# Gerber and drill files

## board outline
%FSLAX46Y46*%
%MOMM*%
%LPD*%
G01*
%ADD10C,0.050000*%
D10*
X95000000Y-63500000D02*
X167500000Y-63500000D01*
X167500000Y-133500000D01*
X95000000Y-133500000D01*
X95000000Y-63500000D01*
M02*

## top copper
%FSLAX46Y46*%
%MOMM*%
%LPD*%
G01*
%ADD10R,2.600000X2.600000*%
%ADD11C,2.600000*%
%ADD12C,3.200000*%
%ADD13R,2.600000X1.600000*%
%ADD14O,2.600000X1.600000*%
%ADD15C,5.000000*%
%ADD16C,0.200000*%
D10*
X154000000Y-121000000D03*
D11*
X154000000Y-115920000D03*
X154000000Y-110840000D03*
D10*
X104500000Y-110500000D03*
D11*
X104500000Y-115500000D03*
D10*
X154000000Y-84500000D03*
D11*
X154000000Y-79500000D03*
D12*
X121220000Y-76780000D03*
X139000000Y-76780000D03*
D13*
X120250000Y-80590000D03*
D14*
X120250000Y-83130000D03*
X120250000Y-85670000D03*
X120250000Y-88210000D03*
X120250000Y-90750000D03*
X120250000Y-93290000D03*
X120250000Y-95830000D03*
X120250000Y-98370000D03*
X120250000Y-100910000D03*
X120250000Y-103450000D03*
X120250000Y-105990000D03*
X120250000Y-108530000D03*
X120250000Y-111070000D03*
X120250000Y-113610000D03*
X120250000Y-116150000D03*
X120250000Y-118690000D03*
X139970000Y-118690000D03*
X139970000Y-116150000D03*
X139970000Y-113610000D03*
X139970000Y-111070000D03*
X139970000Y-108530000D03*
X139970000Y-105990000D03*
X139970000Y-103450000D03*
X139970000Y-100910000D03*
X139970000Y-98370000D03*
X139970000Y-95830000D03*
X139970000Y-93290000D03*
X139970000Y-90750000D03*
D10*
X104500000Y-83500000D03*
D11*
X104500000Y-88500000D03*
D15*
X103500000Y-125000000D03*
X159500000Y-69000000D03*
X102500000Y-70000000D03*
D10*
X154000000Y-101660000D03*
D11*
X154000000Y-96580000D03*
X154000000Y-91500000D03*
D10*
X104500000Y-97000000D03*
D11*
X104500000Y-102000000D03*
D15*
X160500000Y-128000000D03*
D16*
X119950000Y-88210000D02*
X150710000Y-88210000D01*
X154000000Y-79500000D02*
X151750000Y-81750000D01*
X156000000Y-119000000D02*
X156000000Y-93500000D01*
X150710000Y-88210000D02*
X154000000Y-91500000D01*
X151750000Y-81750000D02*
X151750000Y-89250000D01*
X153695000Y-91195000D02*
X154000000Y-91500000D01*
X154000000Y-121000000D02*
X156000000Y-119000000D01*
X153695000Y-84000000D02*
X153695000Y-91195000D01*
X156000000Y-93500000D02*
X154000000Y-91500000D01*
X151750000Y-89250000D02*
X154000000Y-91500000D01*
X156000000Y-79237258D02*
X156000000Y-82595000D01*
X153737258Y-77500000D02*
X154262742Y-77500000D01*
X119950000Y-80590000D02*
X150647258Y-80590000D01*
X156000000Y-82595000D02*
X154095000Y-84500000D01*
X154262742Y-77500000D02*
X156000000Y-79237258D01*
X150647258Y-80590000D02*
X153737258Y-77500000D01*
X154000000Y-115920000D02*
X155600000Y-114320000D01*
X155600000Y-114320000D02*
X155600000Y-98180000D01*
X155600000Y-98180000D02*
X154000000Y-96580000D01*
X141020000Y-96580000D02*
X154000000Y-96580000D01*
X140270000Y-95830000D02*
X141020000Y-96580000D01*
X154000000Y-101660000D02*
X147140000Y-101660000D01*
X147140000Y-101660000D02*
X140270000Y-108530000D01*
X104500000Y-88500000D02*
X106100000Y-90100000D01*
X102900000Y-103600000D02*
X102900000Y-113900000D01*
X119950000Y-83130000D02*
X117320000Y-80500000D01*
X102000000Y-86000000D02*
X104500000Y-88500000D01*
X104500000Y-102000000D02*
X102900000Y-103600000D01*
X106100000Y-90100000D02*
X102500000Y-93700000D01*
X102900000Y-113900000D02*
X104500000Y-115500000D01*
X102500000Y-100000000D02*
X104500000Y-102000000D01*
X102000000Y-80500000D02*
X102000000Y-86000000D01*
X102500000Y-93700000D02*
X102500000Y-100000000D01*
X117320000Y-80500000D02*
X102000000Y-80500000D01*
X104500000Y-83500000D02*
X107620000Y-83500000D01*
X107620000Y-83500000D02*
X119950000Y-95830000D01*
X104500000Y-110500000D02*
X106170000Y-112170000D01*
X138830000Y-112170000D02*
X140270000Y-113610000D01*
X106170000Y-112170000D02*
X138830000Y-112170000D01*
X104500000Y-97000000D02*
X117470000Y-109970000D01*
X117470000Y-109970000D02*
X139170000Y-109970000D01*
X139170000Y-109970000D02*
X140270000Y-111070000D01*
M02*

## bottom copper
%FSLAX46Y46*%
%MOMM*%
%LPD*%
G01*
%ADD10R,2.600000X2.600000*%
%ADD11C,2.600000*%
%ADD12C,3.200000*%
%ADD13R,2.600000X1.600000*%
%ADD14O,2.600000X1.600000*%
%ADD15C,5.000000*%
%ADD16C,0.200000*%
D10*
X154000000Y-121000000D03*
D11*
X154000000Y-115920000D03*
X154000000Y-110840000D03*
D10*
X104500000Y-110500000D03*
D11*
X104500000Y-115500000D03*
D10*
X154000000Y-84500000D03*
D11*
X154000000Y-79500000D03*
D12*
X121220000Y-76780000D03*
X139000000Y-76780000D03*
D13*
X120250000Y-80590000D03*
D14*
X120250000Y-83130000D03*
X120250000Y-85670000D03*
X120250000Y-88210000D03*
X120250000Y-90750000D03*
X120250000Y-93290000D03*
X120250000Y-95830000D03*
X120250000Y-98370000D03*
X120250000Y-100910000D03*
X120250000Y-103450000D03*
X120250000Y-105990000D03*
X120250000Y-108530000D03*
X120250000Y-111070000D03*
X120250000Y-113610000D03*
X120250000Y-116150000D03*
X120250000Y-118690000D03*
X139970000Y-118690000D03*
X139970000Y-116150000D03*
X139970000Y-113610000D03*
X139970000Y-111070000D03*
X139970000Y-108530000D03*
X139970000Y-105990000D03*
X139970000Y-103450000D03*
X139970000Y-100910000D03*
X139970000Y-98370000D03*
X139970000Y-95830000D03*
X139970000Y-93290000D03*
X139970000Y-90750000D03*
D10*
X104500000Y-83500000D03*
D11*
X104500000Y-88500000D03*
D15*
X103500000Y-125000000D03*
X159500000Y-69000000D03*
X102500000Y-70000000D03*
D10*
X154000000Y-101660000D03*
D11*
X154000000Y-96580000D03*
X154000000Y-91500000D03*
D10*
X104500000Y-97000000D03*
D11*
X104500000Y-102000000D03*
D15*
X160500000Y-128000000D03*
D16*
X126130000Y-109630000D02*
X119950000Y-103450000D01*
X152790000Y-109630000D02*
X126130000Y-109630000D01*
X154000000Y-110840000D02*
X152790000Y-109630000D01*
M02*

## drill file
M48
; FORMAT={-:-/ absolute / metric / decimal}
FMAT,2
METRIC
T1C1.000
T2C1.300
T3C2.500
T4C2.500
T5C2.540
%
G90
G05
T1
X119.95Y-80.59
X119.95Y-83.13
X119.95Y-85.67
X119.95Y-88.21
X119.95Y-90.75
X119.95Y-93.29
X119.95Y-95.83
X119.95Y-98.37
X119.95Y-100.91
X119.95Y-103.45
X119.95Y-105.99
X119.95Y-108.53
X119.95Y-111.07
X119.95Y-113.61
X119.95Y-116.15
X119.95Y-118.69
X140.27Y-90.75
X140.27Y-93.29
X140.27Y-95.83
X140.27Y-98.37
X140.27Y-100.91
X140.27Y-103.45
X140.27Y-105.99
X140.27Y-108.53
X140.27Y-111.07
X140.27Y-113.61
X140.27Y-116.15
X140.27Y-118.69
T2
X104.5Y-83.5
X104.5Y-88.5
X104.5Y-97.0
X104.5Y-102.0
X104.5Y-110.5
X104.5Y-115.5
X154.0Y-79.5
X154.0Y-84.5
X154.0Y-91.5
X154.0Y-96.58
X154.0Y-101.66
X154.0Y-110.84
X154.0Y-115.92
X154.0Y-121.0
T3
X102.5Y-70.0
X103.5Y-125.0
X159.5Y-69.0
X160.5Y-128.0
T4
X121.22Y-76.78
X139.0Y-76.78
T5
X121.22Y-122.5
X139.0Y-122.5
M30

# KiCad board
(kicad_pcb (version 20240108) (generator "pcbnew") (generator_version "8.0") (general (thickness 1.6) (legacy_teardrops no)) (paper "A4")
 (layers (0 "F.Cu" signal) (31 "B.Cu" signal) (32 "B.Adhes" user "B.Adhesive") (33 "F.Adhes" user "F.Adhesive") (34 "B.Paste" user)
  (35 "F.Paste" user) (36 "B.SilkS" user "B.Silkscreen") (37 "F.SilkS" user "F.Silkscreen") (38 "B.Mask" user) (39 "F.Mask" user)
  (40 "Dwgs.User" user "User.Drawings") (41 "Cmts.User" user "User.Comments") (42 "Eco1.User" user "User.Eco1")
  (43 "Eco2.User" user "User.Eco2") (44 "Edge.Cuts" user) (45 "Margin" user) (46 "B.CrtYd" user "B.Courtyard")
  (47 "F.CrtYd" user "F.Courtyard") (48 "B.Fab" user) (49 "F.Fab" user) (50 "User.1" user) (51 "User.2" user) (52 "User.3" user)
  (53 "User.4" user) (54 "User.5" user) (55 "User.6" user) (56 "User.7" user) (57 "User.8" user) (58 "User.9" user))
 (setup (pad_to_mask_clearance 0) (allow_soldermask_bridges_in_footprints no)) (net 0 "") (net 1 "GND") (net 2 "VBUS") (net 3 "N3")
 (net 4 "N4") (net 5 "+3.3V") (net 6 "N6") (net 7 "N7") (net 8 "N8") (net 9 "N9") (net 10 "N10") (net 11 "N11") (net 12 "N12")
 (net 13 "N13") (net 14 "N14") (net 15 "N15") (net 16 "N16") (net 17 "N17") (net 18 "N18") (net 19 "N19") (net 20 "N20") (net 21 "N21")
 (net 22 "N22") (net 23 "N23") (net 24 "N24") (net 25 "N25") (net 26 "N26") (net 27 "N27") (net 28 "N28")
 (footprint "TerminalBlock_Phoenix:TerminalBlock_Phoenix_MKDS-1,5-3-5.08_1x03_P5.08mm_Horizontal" (layer "F.Cu") (at 154 121 90)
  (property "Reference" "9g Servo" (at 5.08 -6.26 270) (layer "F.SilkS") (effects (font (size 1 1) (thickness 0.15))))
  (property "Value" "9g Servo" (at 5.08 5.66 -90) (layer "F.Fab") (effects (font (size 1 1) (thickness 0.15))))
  (pad "1" thru_hole rect (at 0 0 90) (size 2.6 2.6) (drill 1.3) (layers "*.Cu" "*.Mask") (remove_unused_layers no) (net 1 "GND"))
  (pad "2" thru_hole circle (at 5.08 0 90) (size 2.6 2.6) (drill 1.3) (layers "*.Cu" "*.Mask") (remove_unused_layers no) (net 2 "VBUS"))
  (pad "3" thru_hole circle (at 10.16 0 90) (size 2.6 2.6) (drill 1.3) (layers "*.Cu" "*.Mask") (remove_unused_layers no) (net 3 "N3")))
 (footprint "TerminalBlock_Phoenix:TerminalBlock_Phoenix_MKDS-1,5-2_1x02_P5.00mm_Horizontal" (layer "F.Cu") (at 104.5 110.5 -90)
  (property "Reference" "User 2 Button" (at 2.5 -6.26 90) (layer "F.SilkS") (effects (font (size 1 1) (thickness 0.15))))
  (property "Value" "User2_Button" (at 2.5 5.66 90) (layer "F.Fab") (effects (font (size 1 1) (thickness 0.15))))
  (pad "1" thru_hole rect (at 0 0 270) (size 2.6 2.6) (drill 1.3) (layers "*.Cu" "*.Mask") (remove_unused_layers no) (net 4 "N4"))
  (pad "2" thru_hole circle (at 5 0 270) (size 2.6 2.6) (drill 1.3) (layers "*.Cu" "*.Mask") (remove_unused_layers no) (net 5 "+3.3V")))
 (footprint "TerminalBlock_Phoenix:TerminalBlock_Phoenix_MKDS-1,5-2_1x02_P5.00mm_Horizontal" (layer "F.Cu") (at 154 84.5 90)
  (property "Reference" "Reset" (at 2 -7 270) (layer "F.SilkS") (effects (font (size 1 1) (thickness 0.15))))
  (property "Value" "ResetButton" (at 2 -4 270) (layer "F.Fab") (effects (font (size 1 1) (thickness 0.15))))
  (pad "1" thru_hole rect (at 0 0 90) (size 2.6 2.6) (drill 1.3) (layers "*.Cu" "*.Mask") (remove_unused_layers no) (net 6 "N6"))
  (pad "2" thru_hole circle (at 5 0 90) (size 2.6 2.6) (drill 1.3) (layers "*.Cu" "*.Mask") (remove_unused_layers no) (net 1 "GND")))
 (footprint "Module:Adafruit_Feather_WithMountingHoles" (layer "F.Cu") (at 119.95 80.59)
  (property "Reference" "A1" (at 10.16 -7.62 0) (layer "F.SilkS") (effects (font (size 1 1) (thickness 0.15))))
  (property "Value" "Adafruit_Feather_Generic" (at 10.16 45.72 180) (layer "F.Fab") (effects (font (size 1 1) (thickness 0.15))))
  (pad "" np_thru_hole circle (at 1.27 -3.81 270) (size 3.2 3.2) (drill 2.5) (layers "*.Cu" "*.Mask"))
  (pad "" np_thru_hole circle (at 1.27 41.91 270) (size 2.54 2.54) (drill 2.54) (layers "*.Cu" "*.Mask"))
  (pad "" np_thru_hole circle (at 19.05 -3.81 270) (size 3.2 3.2) (drill 2.5) (layers "*.Cu" "*.Mask"))
  (pad "" np_thru_hole circle (at 19.05 41.91 270) (size 2.54 2.54) (drill 2.54) (layers "*.Cu" "*.Mask"))
  (pad "1" thru_hole rect (at 0 0) (size 2.6 1.6) (drill 1 (offset 0.3 0)) (layers "*.Cu" "*.Mask") (remove_unused_layers no) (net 6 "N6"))
  (pad "2" thru_hole oval (at 0 2.54) (size 2.6 1.6) (drill 1 (offset 0.3 0)) (layers "*.Cu" "*.Mask") (remove_unused_layers no)
   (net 5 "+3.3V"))
  (pad "3" thru_hole oval (at 0 5.08) (size 2.6 1.6) (drill 1 (offset 0.3 0)) (layers "*.Cu" "*.Mask") (remove_unused_layers no)
   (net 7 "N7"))
  (pad "4" thru_hole oval (at 0 7.62) (size 2.6 1.6) (drill 1 (offset 0.3 0)) (layers "*.Cu" "*.Mask") (remove_unused_layers no)
   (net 1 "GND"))
  (pad "5" thru_hole oval (at 0 10.16) (size 2.6 1.6) (drill 1 (offset 0.3 0)) (layers "*.Cu" "*.Mask") (remove_unused_layers no)
   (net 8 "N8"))
  (pad "6" thru_hole oval (at 0 12.7) (size 2.6 1.6) (drill 1 (offset 0.3 0)) (layers "*.Cu" "*.Mask") (remove_unused_layers no)
   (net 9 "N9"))
  (pad "7" thru_hole oval (at 0 15.24) (size 2.6 1.6) (drill 1 (offset 0.3 0)) (layers "*.Cu" "*.Mask") (remove_unused_layers no)
   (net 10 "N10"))
  (pad "8" thru_hole oval (at 0 17.78) (size 2.6 1.6) (drill 1 (offset 0.3 0)) (layers "*.Cu" "*.Mask") (remove_unused_layers no)
   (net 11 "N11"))
  (pad "9" thru_hole oval (at 0 20.32) (size 2.6 1.6) (drill 1 (offset 0.3 0)) (layers "*.Cu" "*.Mask") (remove_unused_layers no)
   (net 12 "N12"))
  (pad "10" thru_hole oval (at 0 22.86) (size 2.6 1.6) (drill 1 (offset 0.3 0)) (layers "*.Cu" "*.Mask") (remove_unused_layers no)
   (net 3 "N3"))
  (pad "11" thru_hole oval (at 0 25.4) (size 2.6 1.6) (drill 1 (offset 0.3 0)) (layers "*.Cu" "*.Mask") (remove_unused_layers no)
   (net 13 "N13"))
  (pad "12" thru_hole oval (at 0 27.94) (size 2.6 1.6) (drill 1 (offset 0.3 0)) (layers "*.Cu" "*.Mask") (remove_unused_layers no)
   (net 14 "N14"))
  (pad "13" thru_hole oval (at 0 30.48) (size 2.6 1.6) (drill 1 (offset 0.3 0)) (layers "*.Cu" "*.Mask") (remove_unused_layers no)
   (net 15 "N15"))
  (pad "14" thru_hole oval (at 0 33.02) (size 2.6 1.6) (drill 1 (offset 0.3 0)) (layers "*.Cu" "*.Mask") (remove_unused_layers no)
   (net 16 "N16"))
  (pad "15" thru_hole oval (at 0 35.56) (size 2.6 1.6) (drill 1 (offset 0.3 0)) (layers "*.Cu" "*.Mask") (remove_unused_layers no)
   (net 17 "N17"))
  (pad "16" thru_hole oval (at 0 38.1) (size 2.6 1.6) (drill 1 (offset 0.3 0)) (layers "*.Cu" "*.Mask") (remove_unused_layers no)
   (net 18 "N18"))
  (pad "17" thru_hole oval (at 20.32 38.1 180) (size 2.6 1.6) (drill 1 (offset 0.3 0)) (layers "*.Cu" "*.Mask") (remove_unused_layers no)
   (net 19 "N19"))
  (pad "18" thru_hole oval (at 20.32 35.56 180) (size 2.6 1.6) (drill 1 (offset 0.3 0)) (layers "*.Cu" "*.Mask") (remove_unused_layers no)
   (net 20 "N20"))
  (pad "19" thru_hole oval (at 20.32 33.02 180) (size 2.6 1.6) (drill 1 (offset 0.3 0)) (layers "*.Cu" "*.Mask") (remove_unused_layers no)
   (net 4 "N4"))
  (pad "20" thru_hole oval (at 20.32 30.48 180) (size 2.6 1.6) (drill 1 (offset 0.3 0)) (layers "*.Cu" "*.Mask") (remove_unused_layers no)
   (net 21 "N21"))
  (pad "21" thru_hole oval (at 20.32 27.94 180) (size 2.6 1.6) (drill 1 (offset 0.3 0)) (layers "*.Cu" "*.Mask") (remove_unused_layers no)
   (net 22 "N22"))
  (pad "22" thru_hole oval (at 20.32 25.4 180) (size 2.6 1.6) (drill 1 (offset 0.3 0)) (layers "*.Cu" "*.Mask") (remove_unused_layers no)
   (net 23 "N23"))
  (pad "23" thru_hole oval (at 20.32 22.86 180) (size 2.6 1.6) (drill 1 (offset 0.3 0)) (layers "*.Cu" "*.Mask") (remove_unused_layers no)
   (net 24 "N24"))
  (pad "24" thru_hole oval (at 20.32 20.32 180) (size 2.6 1.6) (drill 1 (offset 0.3 0)) (layers "*.Cu" "*.Mask") (remove_unused_layers no)
   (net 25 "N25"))
  (pad "25" thru_hole oval (at 20.32 17.78 180) (size 2.6 1.6) (drill 1 (offset 0.3 0)) (layers "*.Cu" "*.Mask") (remove_unused_layers no)
   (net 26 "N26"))
  (pad "26" thru_hole oval (at 20.32 15.24 180) (size 2.6 1.6) (drill 1 (offset 0.3 0)) (layers "*.Cu" "*.Mask") (remove_unused_layers no)
   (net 2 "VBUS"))
  (pad "27" thru_hole oval (at 20.32 12.7 180) (size 2.6 1.6) (drill 1 (offset 0.3 0)) (layers "*.Cu" "*.Mask") (remove_unused_layers no)
   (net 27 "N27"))
  (pad "28" thru_hole oval (at 20.32 10.16 180) (size 2.6 1.6) (drill 1 (offset 0.3 0)) (layers "*.Cu" "*.Mask") (remove_unused_layers no)
   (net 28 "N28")))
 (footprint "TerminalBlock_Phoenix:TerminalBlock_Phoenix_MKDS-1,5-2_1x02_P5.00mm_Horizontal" (layer "F.Cu") (at 104.5 83.5 -90)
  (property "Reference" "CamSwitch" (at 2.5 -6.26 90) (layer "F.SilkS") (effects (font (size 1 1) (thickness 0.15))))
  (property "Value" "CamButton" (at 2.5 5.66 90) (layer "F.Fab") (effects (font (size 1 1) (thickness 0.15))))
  (pad "1" thru_hole rect (at 0 0 270) (size 2.6 2.6) (drill 1.3) (layers "*.Cu" "*.Mask") (remove_unused_layers no) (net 10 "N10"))
  (pad "2" thru_hole circle (at 5 0 270) (size 2.6 2.6) (drill 1.3) (layers "*.Cu" "*.Mask") (remove_unused_layers no) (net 5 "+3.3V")))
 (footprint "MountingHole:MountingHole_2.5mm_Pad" (layer "F.Cu") (at 103.5 125)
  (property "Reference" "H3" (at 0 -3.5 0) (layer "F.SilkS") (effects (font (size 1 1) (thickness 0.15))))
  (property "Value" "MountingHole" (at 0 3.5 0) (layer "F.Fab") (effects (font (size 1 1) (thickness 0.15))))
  (pad "1" thru_hole circle (at 0 0) (size 5 5) (drill 2.5) (layers "*.Cu" "*.Mask") (remove_unused_layers no)))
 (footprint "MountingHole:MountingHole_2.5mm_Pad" (layer "F.Cu") (at 159.5 69)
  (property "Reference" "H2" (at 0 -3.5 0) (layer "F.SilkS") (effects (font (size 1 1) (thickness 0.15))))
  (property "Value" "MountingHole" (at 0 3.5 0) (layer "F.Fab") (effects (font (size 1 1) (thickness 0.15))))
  (pad "1" thru_hole circle (at 0 0) (size 5 5) (drill 2.5) (layers "*.Cu" "*.Mask") (remove_unused_layers no)))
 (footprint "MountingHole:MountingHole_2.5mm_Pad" (layer "F.Cu") (at 102.5 70)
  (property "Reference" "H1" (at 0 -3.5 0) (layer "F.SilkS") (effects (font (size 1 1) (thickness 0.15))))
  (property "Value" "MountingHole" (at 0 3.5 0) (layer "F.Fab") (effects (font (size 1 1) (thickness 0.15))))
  (pad "1" thru_hole circle (at 0 0) (size 5 5) (drill 2.5) (layers "*.Cu" "*.Mask") (remove_unused_layers no)))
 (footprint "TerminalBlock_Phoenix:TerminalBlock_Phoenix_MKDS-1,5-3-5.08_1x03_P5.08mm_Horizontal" (layer "F.Cu") (at 154 101.66 90)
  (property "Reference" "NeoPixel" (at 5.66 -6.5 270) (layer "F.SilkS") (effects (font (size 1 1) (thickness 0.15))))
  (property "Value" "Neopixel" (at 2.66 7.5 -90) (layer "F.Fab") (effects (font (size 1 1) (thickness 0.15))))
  (pad "1" thru_hole rect (at 0 0 90) (size 2.6 2.6) (drill 1.3) (layers "*.Cu" "*.Mask") (remove_unused_layers no) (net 22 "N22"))
  (pad "2" thru_hole circle (at 5.08 0 90) (size 2.6 2.6) (drill 1.3) (layers "*.Cu" "*.Mask") (remove_unused_layers no) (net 2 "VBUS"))
  (pad "3" thru_hole circle (at 10.16 0 90) (size 2.6 2.6) (drill 1.3) (layers "*.Cu" "*.Mask") (remove_unused_layers no) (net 1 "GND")))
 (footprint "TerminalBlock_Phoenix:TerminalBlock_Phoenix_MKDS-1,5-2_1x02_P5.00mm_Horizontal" (layer "F.Cu") (at 104.5 97 -90)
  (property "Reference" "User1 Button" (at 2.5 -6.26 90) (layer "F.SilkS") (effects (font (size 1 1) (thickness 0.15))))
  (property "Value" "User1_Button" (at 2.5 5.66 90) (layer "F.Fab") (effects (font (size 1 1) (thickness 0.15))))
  (pad "1" thru_hole rect (at 0 0 270) (size 2.6 2.6) (drill 1.3) (layers "*.Cu" "*.Mask") (remove_unused_layers no) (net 21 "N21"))
  (pad "2" thru_hole circle (at 5 0 270) (size 2.6 2.6) (drill 1.3) (layers "*.Cu" "*.Mask") (remove_unused_layers no) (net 5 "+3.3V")))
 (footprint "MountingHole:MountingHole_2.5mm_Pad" (layer "F.Cu") (at 160.5 128)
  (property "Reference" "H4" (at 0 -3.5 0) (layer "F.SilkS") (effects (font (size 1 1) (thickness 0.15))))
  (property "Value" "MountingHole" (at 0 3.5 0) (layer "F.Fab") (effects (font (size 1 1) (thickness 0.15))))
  (pad "1" thru_hole circle (at 0 0) (size 5 5) (drill 2.5) (layers "*.Cu" "*.Mask") (remove_unused_layers no)))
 (gr_rect (start 95 63.5) (end 167.5 133.5) (stroke (width 0.05) (type default)) (fill none) (layer "Edge.Cuts"))
 (segment (start 126.13 109.63) (end 119.95 103.45) (width 0.2) (layer "B.Cu") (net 3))
 (segment (start 152.79 109.63) (end 126.13 109.63) (width 0.2) (layer "B.Cu") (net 3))
 (segment (start 154 110.84) (end 152.79 109.63) (width 0.2) (layer "B.Cu") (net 3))
 (segment (start 119.95 88.21) (end 150.71 88.21) (width 0.2) (layer "F.Cu") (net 1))
 (segment (start 154 79.5) (end 151.75 81.75) (width 0.2) (layer "F.Cu") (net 1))
 (segment (start 156 119) (end 156 93.5) (width 0.2) (layer "F.Cu") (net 1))
 (segment (start 150.71 88.21) (end 154 91.5) (width 0.2) (layer "F.Cu") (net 1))
 (segment (start 151.75 81.75) (end 151.75 89.25) (width 0.2) (layer "F.Cu") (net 1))
 (segment (start 153.695 91.195) (end 154 91.5) (width 0.2) (layer "F.Cu") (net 1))
 (segment (start 154 121) (end 156 119) (width 0.2) (layer "F.Cu") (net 1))
 (segment (start 153.695 84) (end 153.695 91.195) (width 0.2) (layer "F.Cu") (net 1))
 (segment (start 156 93.5) (end 154 91.5) (width 0.2) (layer "F.Cu") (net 1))
 (segment (start 151.75 89.25) (end 154 91.5) (width 0.2) (layer "F.Cu") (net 1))
 (segment (start 156 79.237258) (end 156 82.595) (width 0.2) (layer "F.Cu") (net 6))
 (segment (start 153.737258 77.5) (end 154.262742 77.5) (width 0.2) (layer "F.Cu") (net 6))
 (segment (start 119.95 80.59) (end 150.647258 80.59) (width 0.2) (layer "F.Cu") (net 6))
 (segment (start 156 82.595) (end 154.095 84.5) (width 0.2) (layer "F.Cu") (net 6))
 (segment (start 154.262742 77.5) (end 156 79.237258) (width 0.2) (layer "F.Cu") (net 6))
 (segment (start 150.647258 80.59) (end 153.737258 77.5) (width 0.2) (layer "F.Cu") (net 6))
 (segment (start 154 115.92) (end 155.6 114.32) (width 0.2) (layer "F.Cu") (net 2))
 (segment (start 155.6 114.32) (end 155.6 98.18) (width 0.2) (layer "F.Cu") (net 2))
 (segment (start 155.6 98.18) (end 154 96.58) (width 0.2) (layer "F.Cu") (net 2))
 (segment (start 141.02 96.58) (end 154 96.58) (width 0.2) (layer "F.Cu") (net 2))
 (segment (start 140.27 95.83) (end 141.02 96.58) (width 0.2) (layer "F.Cu") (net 2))
 (segment (start 154 101.66) (end 147.14 101.66) (width 0.2) (layer "F.Cu") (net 22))
 (segment (start 147.14 101.66) (end 140.27 108.53) (width 0.2) (layer "F.Cu") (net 22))
 (segment (start 104.5 88.5) (end 106.1 90.1) (width 0.2) (layer "F.Cu") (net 5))
 (segment (start 102.9 103.6) (end 102.9 113.9) (width 0.2) (layer "F.Cu") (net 5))
 (segment (start 119.95 83.13) (end 117.32 80.5) (width 0.2) (layer "F.Cu") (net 5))
 (segment (start 102 86) (end 104.5 88.5) (width 0.2) (layer "F.Cu") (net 5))
 (segment (start 104.5 102) (end 102.9 103.6) (width 0.2) (layer "F.Cu") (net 5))
 (segment (start 106.1 90.1) (end 102.5 93.7) (width 0.2) (layer "F.Cu") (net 5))
 (segment (start 102.9 113.9) (end 104.5 115.5) (width 0.2) (layer "F.Cu") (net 5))
 (segment (start 102.5 100) (end 104.5 102) (width 0.2) (layer "F.Cu") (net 5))
 (segment (start 102 80.5) (end 102 86) (width 0.2) (layer "F.Cu") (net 5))
 (segment (start 102.5 93.7) (end 102.5 100) (width 0.2) (layer "F.Cu") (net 5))
 (segment (start 117.32 80.5) (end 102 80.5) (width 0.2) (layer "F.Cu") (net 5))
 (segment (start 104.5 83.5) (end 107.62 83.5) (width 0.2) (layer "F.Cu") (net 10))
 (segment (start 107.62 83.5) (end 119.95 95.83) (width 0.2) (layer "F.Cu") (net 10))
 (segment (start 104.5 110.5) (end 106.17 112.17) (width 0.2) (layer "F.Cu") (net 4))
 (segment (start 138.83 112.17) (end 140.27 113.61) (width 0.2) (layer "F.Cu") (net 4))
 (segment (start 106.17 112.17) (end 138.83 112.17) (width 0.2) (layer "F.Cu") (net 4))
 (segment (start 104.5 97) (end 117.47 109.97) (width 0.2) (layer "F.Cu") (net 21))
 (segment (start 117.47 109.97) (end 139.17 109.97) (width 0.2) (layer "F.Cu") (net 21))
 (segment (start 139.17 109.97) (end 140.27 111.07) (width 0.2) (layer "F.Cu") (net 21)))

